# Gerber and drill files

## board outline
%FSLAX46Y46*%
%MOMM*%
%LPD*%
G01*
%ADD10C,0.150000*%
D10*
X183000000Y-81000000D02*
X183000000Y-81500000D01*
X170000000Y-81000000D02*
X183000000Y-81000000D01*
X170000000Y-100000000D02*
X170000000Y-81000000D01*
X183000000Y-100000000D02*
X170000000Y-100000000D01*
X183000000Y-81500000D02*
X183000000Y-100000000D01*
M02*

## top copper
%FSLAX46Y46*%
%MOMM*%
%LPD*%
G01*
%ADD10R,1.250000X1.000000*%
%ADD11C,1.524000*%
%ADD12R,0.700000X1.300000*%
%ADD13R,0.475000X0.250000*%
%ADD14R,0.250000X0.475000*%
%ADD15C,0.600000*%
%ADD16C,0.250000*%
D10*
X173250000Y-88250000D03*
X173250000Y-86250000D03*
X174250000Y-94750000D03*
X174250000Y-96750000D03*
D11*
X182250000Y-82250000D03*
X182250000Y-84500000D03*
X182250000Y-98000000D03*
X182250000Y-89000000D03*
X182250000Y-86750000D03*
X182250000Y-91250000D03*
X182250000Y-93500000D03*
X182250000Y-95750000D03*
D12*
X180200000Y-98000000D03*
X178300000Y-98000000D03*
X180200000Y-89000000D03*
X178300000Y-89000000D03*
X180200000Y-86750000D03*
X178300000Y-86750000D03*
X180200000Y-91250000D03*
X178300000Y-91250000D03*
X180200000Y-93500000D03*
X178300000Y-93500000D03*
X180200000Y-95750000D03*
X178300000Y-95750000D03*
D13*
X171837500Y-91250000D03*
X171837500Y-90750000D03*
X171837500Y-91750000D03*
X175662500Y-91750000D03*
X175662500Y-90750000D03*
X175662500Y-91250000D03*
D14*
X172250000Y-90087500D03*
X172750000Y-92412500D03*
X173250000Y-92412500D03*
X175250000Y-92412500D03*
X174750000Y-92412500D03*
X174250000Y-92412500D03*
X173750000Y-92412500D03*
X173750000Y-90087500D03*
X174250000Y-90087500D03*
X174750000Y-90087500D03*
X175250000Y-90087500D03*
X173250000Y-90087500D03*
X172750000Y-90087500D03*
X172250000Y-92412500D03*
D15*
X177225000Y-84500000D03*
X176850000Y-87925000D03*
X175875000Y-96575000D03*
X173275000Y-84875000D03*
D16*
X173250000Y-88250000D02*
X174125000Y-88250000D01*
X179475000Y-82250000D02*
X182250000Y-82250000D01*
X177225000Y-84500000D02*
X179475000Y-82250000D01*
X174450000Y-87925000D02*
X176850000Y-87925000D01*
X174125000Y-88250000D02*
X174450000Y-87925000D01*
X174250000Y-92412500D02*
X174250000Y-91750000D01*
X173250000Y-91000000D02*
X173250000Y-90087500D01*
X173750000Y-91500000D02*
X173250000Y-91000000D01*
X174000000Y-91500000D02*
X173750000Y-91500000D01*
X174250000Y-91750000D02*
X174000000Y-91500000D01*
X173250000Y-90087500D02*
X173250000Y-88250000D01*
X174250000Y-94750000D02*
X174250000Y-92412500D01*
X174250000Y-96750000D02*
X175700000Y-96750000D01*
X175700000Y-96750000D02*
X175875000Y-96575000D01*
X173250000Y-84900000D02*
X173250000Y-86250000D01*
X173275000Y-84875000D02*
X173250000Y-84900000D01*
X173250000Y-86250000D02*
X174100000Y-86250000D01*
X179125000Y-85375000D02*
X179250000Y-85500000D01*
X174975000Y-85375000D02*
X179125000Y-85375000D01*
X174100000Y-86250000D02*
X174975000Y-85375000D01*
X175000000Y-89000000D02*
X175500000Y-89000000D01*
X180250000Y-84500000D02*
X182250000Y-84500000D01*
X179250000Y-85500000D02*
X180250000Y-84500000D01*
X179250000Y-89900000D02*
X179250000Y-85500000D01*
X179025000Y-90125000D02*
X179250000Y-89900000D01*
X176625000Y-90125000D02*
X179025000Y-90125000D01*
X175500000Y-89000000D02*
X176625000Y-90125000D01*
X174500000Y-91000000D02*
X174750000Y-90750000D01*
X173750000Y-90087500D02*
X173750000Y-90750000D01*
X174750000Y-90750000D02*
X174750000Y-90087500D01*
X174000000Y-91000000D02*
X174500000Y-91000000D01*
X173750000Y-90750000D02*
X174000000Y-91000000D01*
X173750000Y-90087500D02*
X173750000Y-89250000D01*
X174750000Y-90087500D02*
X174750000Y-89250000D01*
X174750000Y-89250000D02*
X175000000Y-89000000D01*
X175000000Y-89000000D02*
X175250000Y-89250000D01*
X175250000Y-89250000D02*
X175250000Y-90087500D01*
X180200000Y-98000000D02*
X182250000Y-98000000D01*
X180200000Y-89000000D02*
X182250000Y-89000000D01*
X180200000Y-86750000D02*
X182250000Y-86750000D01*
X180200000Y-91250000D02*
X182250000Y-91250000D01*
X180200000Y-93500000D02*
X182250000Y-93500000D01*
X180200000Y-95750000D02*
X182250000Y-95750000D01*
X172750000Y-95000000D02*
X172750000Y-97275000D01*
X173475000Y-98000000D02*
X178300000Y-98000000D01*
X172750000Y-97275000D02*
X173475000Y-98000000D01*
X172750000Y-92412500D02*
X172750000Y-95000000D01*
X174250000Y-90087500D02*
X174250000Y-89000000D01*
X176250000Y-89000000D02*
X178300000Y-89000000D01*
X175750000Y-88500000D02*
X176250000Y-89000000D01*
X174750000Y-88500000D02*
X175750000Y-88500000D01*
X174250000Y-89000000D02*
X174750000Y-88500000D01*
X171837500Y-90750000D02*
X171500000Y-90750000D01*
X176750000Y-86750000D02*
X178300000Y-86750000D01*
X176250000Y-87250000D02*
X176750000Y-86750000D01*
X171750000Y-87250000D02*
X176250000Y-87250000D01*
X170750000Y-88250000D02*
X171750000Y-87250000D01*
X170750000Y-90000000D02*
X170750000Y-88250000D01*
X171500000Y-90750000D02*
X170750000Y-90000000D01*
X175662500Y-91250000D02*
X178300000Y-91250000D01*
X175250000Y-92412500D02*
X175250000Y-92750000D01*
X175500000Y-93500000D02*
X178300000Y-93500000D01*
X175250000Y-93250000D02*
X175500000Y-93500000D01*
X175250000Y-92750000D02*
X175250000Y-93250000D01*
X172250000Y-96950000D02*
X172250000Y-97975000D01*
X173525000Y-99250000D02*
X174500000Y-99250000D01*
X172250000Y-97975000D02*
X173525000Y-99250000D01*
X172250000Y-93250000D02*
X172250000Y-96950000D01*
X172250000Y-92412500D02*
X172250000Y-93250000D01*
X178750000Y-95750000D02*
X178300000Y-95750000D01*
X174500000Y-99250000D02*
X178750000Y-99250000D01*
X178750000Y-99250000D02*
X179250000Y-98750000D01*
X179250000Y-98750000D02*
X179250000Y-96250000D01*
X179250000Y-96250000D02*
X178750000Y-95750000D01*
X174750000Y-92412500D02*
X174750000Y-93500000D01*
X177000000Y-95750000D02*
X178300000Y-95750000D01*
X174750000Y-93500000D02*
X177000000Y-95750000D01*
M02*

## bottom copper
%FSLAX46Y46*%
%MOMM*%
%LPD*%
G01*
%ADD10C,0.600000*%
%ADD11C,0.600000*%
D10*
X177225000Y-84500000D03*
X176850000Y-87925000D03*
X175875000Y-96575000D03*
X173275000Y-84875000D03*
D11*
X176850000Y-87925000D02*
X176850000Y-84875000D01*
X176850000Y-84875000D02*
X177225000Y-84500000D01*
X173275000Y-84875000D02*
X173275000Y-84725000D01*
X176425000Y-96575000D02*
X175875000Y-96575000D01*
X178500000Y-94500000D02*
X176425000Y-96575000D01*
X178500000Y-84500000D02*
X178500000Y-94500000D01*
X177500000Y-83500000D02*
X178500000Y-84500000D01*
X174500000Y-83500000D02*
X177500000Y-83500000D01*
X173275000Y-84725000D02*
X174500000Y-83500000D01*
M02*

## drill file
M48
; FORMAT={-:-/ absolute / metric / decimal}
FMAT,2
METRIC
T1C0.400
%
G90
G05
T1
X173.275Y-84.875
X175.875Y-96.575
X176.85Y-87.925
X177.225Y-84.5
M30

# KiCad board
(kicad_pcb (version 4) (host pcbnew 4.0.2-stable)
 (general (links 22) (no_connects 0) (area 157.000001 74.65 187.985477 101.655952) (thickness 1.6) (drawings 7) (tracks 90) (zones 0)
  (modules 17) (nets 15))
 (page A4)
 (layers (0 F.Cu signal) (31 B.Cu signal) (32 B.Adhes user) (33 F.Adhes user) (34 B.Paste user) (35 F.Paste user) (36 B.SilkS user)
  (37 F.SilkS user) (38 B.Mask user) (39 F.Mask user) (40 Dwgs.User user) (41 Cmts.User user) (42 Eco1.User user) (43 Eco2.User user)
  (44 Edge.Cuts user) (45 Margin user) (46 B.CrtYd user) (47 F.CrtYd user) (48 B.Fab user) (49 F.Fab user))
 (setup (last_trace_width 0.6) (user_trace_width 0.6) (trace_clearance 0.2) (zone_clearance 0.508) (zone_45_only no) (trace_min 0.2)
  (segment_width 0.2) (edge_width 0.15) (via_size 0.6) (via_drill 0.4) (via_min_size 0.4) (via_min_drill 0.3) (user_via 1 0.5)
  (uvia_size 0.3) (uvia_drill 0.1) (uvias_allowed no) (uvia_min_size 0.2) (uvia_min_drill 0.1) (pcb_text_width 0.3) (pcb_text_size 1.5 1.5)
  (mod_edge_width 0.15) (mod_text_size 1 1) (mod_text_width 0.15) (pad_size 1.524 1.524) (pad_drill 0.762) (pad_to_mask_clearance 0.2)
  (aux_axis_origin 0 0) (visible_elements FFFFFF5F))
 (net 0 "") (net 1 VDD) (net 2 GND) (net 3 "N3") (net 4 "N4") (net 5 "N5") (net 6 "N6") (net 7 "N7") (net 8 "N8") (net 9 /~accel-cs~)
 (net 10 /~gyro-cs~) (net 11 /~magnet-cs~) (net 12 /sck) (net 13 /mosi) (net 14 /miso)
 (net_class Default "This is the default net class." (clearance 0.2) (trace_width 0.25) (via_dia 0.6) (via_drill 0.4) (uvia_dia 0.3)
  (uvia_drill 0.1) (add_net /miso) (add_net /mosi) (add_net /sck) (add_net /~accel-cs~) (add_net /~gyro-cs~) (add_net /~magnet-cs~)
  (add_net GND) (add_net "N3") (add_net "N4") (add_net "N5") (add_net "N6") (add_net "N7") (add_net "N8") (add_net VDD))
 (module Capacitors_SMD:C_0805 (layer F.Cu) (at 173.25 87.25 90)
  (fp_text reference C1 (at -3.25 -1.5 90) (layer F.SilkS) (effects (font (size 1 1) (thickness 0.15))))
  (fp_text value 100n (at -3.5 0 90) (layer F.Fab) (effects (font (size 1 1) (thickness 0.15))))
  (pad 1 smd rect (at -1 0 90) (size 1 1.25) (layers F.Cu F.Paste F.Mask) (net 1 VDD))
  (pad 2 smd rect (at 1 0 90) (size 1 1.25) (layers F.Cu F.Paste F.Mask) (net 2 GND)))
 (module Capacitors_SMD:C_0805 (layer F.Cu) (at 174.25 95.75 270)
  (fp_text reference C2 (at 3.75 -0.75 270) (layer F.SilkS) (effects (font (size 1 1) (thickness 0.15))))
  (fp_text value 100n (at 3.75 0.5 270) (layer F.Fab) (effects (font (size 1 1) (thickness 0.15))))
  (pad 1 smd rect (at -1 0 270) (size 1 1.25) (layers F.Cu F.Paste F.Mask) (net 1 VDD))
  (pad 2 smd rect (at 1 0 270) (size 1 1.25) (layers F.Cu F.Paste F.Mask) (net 2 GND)))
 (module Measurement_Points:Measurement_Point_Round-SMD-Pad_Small (layer F.Cu) (at 182.25 82.25)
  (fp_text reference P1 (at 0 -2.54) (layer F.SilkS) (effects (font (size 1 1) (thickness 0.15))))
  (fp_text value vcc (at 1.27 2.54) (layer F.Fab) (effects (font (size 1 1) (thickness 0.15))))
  (pad 1 smd circle (at 0 0) (size 1.524 1.524) (layers F.Cu F.Paste F.Mask) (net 1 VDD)))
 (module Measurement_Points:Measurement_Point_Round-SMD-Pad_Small (layer F.Cu) (at 182.25 84.5)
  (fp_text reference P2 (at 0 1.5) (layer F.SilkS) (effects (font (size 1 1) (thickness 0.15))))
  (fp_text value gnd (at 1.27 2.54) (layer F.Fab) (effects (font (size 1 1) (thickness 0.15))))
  (pad 1 smd circle (at 0 0) (size 1.524 1.524) (layers F.Cu F.Paste F.Mask) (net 2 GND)))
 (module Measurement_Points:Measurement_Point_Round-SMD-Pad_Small (layer F.Cu) (at 182.25 98)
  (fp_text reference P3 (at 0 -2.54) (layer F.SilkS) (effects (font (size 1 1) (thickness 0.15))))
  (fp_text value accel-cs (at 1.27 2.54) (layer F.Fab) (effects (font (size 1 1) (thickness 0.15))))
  (pad 1 smd circle (at 0 0) (size 1.524 1.524) (layers F.Cu F.Paste F.Mask) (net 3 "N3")))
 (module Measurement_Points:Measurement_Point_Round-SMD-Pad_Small (layer F.Cu) (at 182.25 89)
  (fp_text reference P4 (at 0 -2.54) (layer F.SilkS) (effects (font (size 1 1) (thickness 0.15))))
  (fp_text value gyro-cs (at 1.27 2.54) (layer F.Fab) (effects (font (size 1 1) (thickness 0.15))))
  (pad 1 smd circle (at 0 0) (size 1.524 1.524) (layers F.Cu F.Paste F.Mask) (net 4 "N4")))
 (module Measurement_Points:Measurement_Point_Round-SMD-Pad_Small (layer F.Cu) (at 182.25 86.75)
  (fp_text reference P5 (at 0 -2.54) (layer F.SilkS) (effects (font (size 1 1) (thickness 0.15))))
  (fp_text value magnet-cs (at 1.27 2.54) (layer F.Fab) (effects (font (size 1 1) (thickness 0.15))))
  (pad 1 smd circle (at 0 0) (size 1.524 1.524) (layers F.Cu F.Paste F.Mask) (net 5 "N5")))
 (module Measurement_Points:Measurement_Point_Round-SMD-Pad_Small (layer F.Cu) (at 182.25 91.25)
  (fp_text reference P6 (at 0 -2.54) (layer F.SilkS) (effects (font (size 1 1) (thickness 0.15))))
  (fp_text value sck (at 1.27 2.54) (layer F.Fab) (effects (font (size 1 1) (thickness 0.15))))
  (pad 1 smd circle (at 0 0) (size 1.524 1.524) (layers F.Cu F.Paste F.Mask) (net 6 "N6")))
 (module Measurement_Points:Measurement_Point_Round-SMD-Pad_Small (layer F.Cu) (at 182.25 93.5)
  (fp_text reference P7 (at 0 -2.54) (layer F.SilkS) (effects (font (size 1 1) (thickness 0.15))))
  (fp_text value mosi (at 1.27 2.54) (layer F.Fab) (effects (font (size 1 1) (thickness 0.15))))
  (pad 1 smd circle (at 0 0) (size 1.524 1.524) (layers F.Cu F.Paste F.Mask) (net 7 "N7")))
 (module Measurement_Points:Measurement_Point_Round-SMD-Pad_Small (layer F.Cu) (at 182.25 95.75)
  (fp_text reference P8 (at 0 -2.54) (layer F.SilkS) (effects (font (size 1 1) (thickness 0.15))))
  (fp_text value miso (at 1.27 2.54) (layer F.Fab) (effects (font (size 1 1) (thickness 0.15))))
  (pad 1 smd circle (at 0 0) (size 1.524 1.524) (layers F.Cu F.Paste F.Mask) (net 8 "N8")))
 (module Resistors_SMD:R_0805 (layer F.Cu) (at 179.25 98 180)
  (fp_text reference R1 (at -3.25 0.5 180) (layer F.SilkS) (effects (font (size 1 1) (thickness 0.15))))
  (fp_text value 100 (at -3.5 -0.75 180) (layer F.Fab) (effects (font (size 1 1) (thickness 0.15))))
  (pad 1 smd rect (at -0.95 0 180) (size 0.7 1.3) (layers F.Cu F.Paste F.Mask) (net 3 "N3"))
  (pad 2 smd rect (at 0.95 0 180) (size 0.7 1.3) (layers F.Cu F.Paste F.Mask) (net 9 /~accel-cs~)))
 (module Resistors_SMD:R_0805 (layer F.Cu) (at 179.25 89 180)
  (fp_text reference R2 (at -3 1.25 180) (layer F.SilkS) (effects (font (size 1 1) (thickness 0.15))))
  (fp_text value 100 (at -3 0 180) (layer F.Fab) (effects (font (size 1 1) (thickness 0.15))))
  (pad 1 smd rect (at -0.95 0 180) (size 0.7 1.3) (layers F.Cu F.Paste F.Mask) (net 4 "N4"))
  (pad 2 smd rect (at 0.95 0 180) (size 0.7 1.3) (layers F.Cu F.Paste F.Mask) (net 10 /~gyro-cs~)))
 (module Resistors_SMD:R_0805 (layer F.Cu) (at 179.25 86.75 180)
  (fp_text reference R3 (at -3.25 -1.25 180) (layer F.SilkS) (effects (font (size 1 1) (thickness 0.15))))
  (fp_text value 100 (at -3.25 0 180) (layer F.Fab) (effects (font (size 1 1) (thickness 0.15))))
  (pad 1 smd rect (at -0.95 0 180) (size 0.7 1.3) (layers F.Cu F.Paste F.Mask) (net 5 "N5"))
  (pad 2 smd rect (at 0.95 0 180) (size 0.7 1.3) (layers F.Cu F.Paste F.Mask) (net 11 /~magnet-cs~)))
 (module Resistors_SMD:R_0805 (layer F.Cu) (at 179.25 91.25 180)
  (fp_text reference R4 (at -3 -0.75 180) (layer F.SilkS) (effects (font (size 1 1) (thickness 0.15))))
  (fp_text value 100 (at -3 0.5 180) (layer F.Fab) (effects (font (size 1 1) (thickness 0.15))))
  (pad 1 smd rect (at -0.95 0 180) (size 0.7 1.3) (layers F.Cu F.Paste F.Mask) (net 6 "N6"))
  (pad 2 smd rect (at 0.95 0 180) (size 0.7 1.3) (layers F.Cu F.Paste F.Mask) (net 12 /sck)))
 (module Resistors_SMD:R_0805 (layer F.Cu) (at 179.25 93.5 180)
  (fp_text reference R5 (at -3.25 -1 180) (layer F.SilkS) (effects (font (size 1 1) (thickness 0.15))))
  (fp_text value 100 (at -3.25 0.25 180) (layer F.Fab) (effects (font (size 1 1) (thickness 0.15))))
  (pad 1 smd rect (at -0.95 0 180) (size 0.7 1.3) (layers F.Cu F.Paste F.Mask) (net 7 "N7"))
  (pad 2 smd rect (at 0.95 0 180) (size 0.7 1.3) (layers F.Cu F.Paste F.Mask) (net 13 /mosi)))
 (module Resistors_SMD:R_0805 (layer F.Cu) (at 179.25 95.75 180)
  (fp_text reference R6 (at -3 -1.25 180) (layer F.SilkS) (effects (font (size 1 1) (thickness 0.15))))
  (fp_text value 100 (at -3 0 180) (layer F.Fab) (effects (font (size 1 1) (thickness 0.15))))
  (pad 1 smd rect (at -0.95 0 180) (size 0.7 1.3) (layers F.Cu F.Paste F.Mask) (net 8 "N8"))
  (pad 2 smd rect (at 0.95 0 180) (size 0.7 1.3) (layers F.Cu F.Paste F.Mask) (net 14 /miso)))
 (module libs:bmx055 (layer F.Cu) (at 173.75 91.25)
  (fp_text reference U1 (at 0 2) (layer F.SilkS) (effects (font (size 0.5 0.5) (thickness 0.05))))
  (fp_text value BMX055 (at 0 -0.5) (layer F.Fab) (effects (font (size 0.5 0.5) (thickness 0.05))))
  (pad 19 smd rect (at -1.9125 0) (size 0.475 0.25) (layers F.Cu F.Paste F.Mask))
  (pad 20 smd rect (at -1.9125 -0.5) (size 0.475 0.25) (layers F.Cu F.Paste F.Mask) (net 11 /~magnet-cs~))
  (pad 18 smd rect (at -1.9125 0.5) (size 0.475 0.25) (layers F.Cu F.Paste F.Mask))
  (pad 10 smd rect (at 1.9125 0.5) (size 0.475 0.25) (layers F.Cu F.Paste F.Mask))
  (pad 8 smd rect (at 1.9125 -0.5) (size 0.475 0.25) (layers F.Cu F.Paste F.Mask))
  (pad 9 smd rect (at 1.9125 0) (size 0.475 0.25) (layers F.Cu F.Paste F.Mask) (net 12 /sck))
  (pad 1 smd rect (at -1.5 -1.1625) (size 0.25 0.475) (layers F.Cu F.Paste F.Mask))
  (pad 16 smd rect (at -1 1.1625) (size 0.25 0.475) (layers F.Cu F.Paste F.Mask) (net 9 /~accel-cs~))
  (pad 15 smd rect (at -0.5 1.1625) (size 0.25 0.475) (layers F.Cu F.Paste F.Mask))
  (pad 11 smd rect (at 1.5 1.1625) (size 0.25 0.475) (layers F.Cu F.Paste F.Mask) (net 13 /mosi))
  (pad 12 smd rect (at 1 1.1625) (size 0.25 0.475) (layers F.Cu F.Paste F.Mask) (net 14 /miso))
  (pad 13 smd rect (at 0.5 1.1625) (size 0.25 0.475) (layers F.Cu F.Paste F.Mask) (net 1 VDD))
  (pad 14 smd rect (at 0 1.1625) (size 0.25 0.475) (layers F.Cu F.Paste F.Mask))
  (pad 4 smd rect (at 0 -1.1625) (size 0.25 0.475) (layers F.Cu F.Paste F.Mask) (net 2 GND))
  (pad 5 smd rect (at 0.5 -1.1625) (size 0.25 0.475) (layers F.Cu F.Paste F.Mask) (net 10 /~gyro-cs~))
  (pad 6 smd rect (at 1 -1.1625) (size 0.25 0.475) (layers F.Cu F.Paste F.Mask) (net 2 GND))
  (pad 7 smd rect (at 1.5 -1.1625) (size 0.25 0.475) (layers F.Cu F.Paste F.Mask) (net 2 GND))
  (pad 3 smd rect (at -0.5 -1.1625) (size 0.25 0.475) (layers F.Cu F.Paste F.Mask) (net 1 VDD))
  (pad 2 smd rect (at -1 -1.1625) (size 0.25 0.475) (layers F.Cu F.Paste F.Mask))
  (pad 17 smd rect (at -1.5 1.1625) (size 0.25 0.475) (layers F.Cu F.Paste F.Mask) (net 14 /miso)))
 (gr_line (start 183 81) (end 183 81.5) (angle 90) (layer Edge.Cuts) (width 0.15))
 (gr_line (start 170 81) (end 183 81) (angle 90) (layer Edge.Cuts) (width 0.15))
 (gr_line (start 170 100) (end 170 81) (angle 90) (layer Edge.Cuts) (width 0.15))
 (gr_line (start 183 100) (end 170 100) (angle 90) (layer Edge.Cuts) (width 0.15))
 (gr_line (start 183 81.5) (end 183 100) (angle 90) (layer Edge.Cuts) (width 0.15))
 (segment (start 176.85 87.925) (end 176.85 84.875) (width 0.6) (layer B.Cu) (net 1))
 (segment (start 176.85 84.875) (end 177.225 84.5) (width 0.6) (layer B.Cu) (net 1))
 (segment (start 173.25 88.25) (end 174.125 88.25) (width 0.25) (layer F.Cu) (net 1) (status 400000))
 (segment (start 179.475 82.25) (end 182.25 82.25) (width 0.25) (layer F.Cu) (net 1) (status 800000))
 (via (at 177.225 84.5) (size 0.6) (drill 0.4) (layers F.Cu B.Cu) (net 1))
 (segment (start 177.225 84.5) (end 179.475 82.25) (width 0.25) (layer F.Cu) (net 1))
 (via (at 176.85 87.925) (size 0.6) (drill 0.4) (layers F.Cu B.Cu) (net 1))
 (segment (start 174.45 87.925) (end 176.85 87.925) (width 0.25) (layer F.Cu) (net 1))
 (segment (start 174.125 88.25) (end 174.45 87.925) (width 0.25) (layer F.Cu) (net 1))
 (segment (start 174.25 92.4125) (end 174.25 91.75) (width 0.25) (layer F.Cu) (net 1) (status 400000))
 (segment (start 173.25 91) (end 173.25 90.0875) (width 0.25) (layer F.Cu) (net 1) (status 800000))
 (segment (start 173.75 91.5) (end 173.25 91) (width 0.25) (layer F.Cu) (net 1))
 (segment (start 174 91.5) (end 173.75 91.5) (width 0.25) (layer F.Cu) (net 1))
 (segment (start 174.25 91.75) (end 174 91.5) (width 0.25) (layer F.Cu) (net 1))
 (segment (start 173.25 90.0875) (end 173.25 88.25) (width 0.25) (layer F.Cu) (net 1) (status C00000))
 (segment (start 174.25 94.75) (end 174.25 92.4125) (width 0.25) (layer F.Cu) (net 1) (status C00000))
 (segment (start 173.275 84.875) (end 173.275 84.725) (width 0.6) (layer B.Cu) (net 2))
 (segment (start 176.425 96.575) (end 175.875 96.575) (width 0.6) (layer B.Cu) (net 2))
 (segment (start 178.5 94.5) (end 176.425 96.575) (width 0.6) (layer B.Cu) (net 2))
 (segment (start 178.5 84.5) (end 178.5 94.5) (width 0.6) (layer B.Cu) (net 2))
 (segment (start 177.5 83.5) (end 178.5 84.5) (width 0.6) (layer B.Cu) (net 2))
 (segment (start 174.5 83.5) (end 177.5 83.5) (width 0.6) (layer B.Cu) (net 2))
 (segment (start 173.275 84.725) (end 174.5 83.5) (width 0.6) (layer B.Cu) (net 2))
 (segment (start 174.25 96.75) (end 175.7 96.75) (width 0.25) (layer F.Cu) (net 2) (status 400000))
 (segment (start 175.7 96.75) (end 175.875 96.575) (width 0.25) (layer F.Cu) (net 2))
 (via (at 175.875 96.575) (size 0.6) (drill 0.4) (layers F.Cu B.Cu) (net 2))
 (segment (start 173.25 84.9) (end 173.25 86.25) (width 0.25) (layer F.Cu) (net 2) (status 800000))
 (segment (start 173.275 84.875) (end 173.25 84.9) (width 0.25) (layer F.Cu) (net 2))
 (via (at 173.275 84.875) (size 0.6) (drill 0.4) (layers F.Cu B.Cu) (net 2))
 (segment (start 173.25 86.25) (end 174.1 86.25) (width 0.25) (layer F.Cu) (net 2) (status 400000))
 (segment (start 179.125 85.375) (end 179.25 85.5) (width 0.25) (layer F.Cu) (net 2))
 (segment (start 174.975 85.375) (end 179.125 85.375) (width 0.25) (layer F.Cu) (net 2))
 (segment (start 174.1 86.25) (end 174.975 85.375) (width 0.25) (layer F.Cu) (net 2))
 (segment (start 175 89) (end 175.5 89) (width 0.25) (layer F.Cu) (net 2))
 (segment (start 180.25 84.5) (end 182.25 84.5) (width 0.25) (layer F.Cu) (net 2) (status 800000))
 (segment (start 179.25 85.5) (end 180.25 84.5) (width 0.25) (layer F.Cu) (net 2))
 (segment (start 179.25 89.9) (end 179.25 85.5) (width 0.25) (layer F.Cu) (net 2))
 (segment (start 179.025 90.125) (end 179.25 89.9) (width 0.25) (layer F.Cu) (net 2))
 (segment (start 176.625 90.125) (end 179.025 90.125) (width 0.25) (layer F.Cu) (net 2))
 (segment (start 175.5 89) (end 176.625 90.125) (width 0.25) (layer F.Cu) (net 2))
 (segment (start 174.5 91) (end 174.75 90.75) (width 0.25) (layer F.Cu) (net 2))
 (segment (start 173.75 90.0875) (end 173.75 90.75) (width 0.25) (layer F.Cu) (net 2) (status 400000))
 (segment (start 174.75 90.75) (end 174.75 90.0875) (width 0.25) (layer F.Cu) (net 2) (status 800000))
 (segment (start 174 91) (end 174.5 91) (width 0.25) (layer F.Cu) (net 2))
 (segment (start 173.75 90.75) (end 174 91) (width 0.25) (layer F.Cu) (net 2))
 (segment (start 173.75 90.0875) (end 173.75 89.25) (width 0.25) (layer F.Cu) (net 2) (status 400000))
 (segment (start 174.75 90.0875) (end 174.75 89.25) (width 0.25) (layer F.Cu) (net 2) (status 400000))
 (segment (start 174.75 89.25) (end 175 89) (width 0.25) (layer F.Cu) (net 2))
 (segment (start 175 89) (end 175.25 89.25) (width 0.25) (layer F.Cu) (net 2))
 (segment (start 175.25 89.25) (end 175.25 90.0875) (width 0.25) (layer F.Cu) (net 2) (status 800000))
 (segment (start 180.2 98) (end 182.25 98) (width 0.25) (layer F.Cu) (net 3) (status C00000))
 (segment (start 180.2 89) (end 182.25 89) (width 0.25) (layer F.Cu) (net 4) (status C00000))
 (segment (start 180.2 86.75) (end 182.25 86.75) (width 0.25) (layer F.Cu) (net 5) (status C00000))
 (segment (start 180.2 91.25) (end 182.25 91.25) (width 0.25) (layer F.Cu) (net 6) (status C00000))
 (segment (start 180.2 93.5) (end 182.25 93.5) (width 0.25) (layer F.Cu) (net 7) (status C00000))
 (segment (start 180.2 95.75) (end 182.25 95.75) (width 0.25) (layer F.Cu) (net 8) (status C00000))
 (segment (start 172.75 95) (end 172.75 97.275) (width 0.25) (layer F.Cu) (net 9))
 (segment (start 173.475 98) (end 178.3 98) (width 0.25) (layer F.Cu) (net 9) (status 800000))
 (segment (start 172.75 97.275) (end 173.475 98) (width 0.25) (layer F.Cu) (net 9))
 (segment (start 172.75 92.4125) (end 172.75 95) (width 0.25) (layer F.Cu) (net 9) (status 400000))
 (segment (start 174.25 90.0875) (end 174.25 89) (width 0.25) (layer F.Cu) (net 10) (status 400000))
 (segment (start 176.25 89) (end 178.3 89) (width 0.25) (layer F.Cu) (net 10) (status 800000))
 (segment (start 175.75 88.5) (end 176.25 89) (width 0.25) (layer F.Cu) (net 10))
 (segment (start 174.75 88.5) (end 175.75 88.5) (width 0.25) (layer F.Cu) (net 10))
 (segment (start 174.25 89) (end 174.75 88.5) (width 0.25) (layer F.Cu) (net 10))
 (segment (start 171.8375 90.75) (end 171.5 90.75) (width 0.25) (layer F.Cu) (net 11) (status 400000))
 (segment (start 176.75 86.75) (end 178.3 86.75) (width 0.25) (layer F.Cu) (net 11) (status 800000))
 (segment (start 176.25 87.25) (end 176.75 86.75) (width 0.25) (layer F.Cu) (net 11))
 (segment (start 171.75 87.25) (end 176.25 87.25) (width 0.25) (layer F.Cu) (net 11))
 (segment (start 170.75 88.25) (end 171.75 87.25) (width 0.25) (layer F.Cu) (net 11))
 (segment (start 170.75 90) (end 170.75 88.25) (width 0.25) (layer F.Cu) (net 11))
 (segment (start 171.5 90.75) (end 170.75 90) (width 0.25) (layer F.Cu) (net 11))
 (segment (start 175.6625 91.25) (end 178.3 91.25) (width 0.25) (layer F.Cu) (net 12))
 (segment (start 175.25 92.4125) (end 175.25 92.75) (width 0.25) (layer F.Cu) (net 13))
 (segment (start 175.5 93.5) (end 178.3 93.5) (width 0.25) (layer F.Cu) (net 13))
 (segment (start 175.25 93.25) (end 175.5 93.5) (width 0.25) (layer F.Cu) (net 13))
 (segment (start 175.25 92.75) (end 175.25 93.25) (width 0.25) (layer F.Cu) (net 13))
 (segment (start 172.25 96.95) (end 172.25 97.975) (width 0.25) (layer F.Cu) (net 14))
 (segment (start 173.525 99.25) (end 174.5 99.25) (width 0.25) (layer F.Cu) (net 14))
 (segment (start 172.25 97.975) (end 173.525 99.25) (width 0.25) (layer F.Cu) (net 14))
 (segment (start 172.25 93.25) (end 172.25 96.95) (width 0.25) (layer F.Cu) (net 14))
 (segment (start 172.25 92.4125) (end 172.25 93.25) (width 0.25) (layer F.Cu) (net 14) (status 400000))
 (segment (start 178.75 95.75) (end 178.3 95.75) (width 0.25) (layer F.Cu) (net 14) (status 800000))
 (segment (start 174.5 99.25) (end 178.75 99.25) (width 0.25) (layer F.Cu) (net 14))
 (segment (start 178.75 99.25) (end 179.25 98.75) (width 0.25) (layer F.Cu) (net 14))
 (segment (start 179.25 98.75) (end 179.25 96.25) (width 0.25) (layer F.Cu) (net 14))
 (segment (start 179.25 96.25) (end 178.75 95.75) (width 0.25) (layer F.Cu) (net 14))
 (segment (start 174.75 92.4125) (end 174.75 93.5) (width 0.25) (layer F.Cu) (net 14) (status 400000))
 (segment (start 177 95.75) (end 178.3 95.75) (width 0.25) (layer F.Cu) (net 14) (status 800000))
 (segment (start 174.75 93.5) (end 177 95.75) (width 0.25) (layer F.Cu) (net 14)))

